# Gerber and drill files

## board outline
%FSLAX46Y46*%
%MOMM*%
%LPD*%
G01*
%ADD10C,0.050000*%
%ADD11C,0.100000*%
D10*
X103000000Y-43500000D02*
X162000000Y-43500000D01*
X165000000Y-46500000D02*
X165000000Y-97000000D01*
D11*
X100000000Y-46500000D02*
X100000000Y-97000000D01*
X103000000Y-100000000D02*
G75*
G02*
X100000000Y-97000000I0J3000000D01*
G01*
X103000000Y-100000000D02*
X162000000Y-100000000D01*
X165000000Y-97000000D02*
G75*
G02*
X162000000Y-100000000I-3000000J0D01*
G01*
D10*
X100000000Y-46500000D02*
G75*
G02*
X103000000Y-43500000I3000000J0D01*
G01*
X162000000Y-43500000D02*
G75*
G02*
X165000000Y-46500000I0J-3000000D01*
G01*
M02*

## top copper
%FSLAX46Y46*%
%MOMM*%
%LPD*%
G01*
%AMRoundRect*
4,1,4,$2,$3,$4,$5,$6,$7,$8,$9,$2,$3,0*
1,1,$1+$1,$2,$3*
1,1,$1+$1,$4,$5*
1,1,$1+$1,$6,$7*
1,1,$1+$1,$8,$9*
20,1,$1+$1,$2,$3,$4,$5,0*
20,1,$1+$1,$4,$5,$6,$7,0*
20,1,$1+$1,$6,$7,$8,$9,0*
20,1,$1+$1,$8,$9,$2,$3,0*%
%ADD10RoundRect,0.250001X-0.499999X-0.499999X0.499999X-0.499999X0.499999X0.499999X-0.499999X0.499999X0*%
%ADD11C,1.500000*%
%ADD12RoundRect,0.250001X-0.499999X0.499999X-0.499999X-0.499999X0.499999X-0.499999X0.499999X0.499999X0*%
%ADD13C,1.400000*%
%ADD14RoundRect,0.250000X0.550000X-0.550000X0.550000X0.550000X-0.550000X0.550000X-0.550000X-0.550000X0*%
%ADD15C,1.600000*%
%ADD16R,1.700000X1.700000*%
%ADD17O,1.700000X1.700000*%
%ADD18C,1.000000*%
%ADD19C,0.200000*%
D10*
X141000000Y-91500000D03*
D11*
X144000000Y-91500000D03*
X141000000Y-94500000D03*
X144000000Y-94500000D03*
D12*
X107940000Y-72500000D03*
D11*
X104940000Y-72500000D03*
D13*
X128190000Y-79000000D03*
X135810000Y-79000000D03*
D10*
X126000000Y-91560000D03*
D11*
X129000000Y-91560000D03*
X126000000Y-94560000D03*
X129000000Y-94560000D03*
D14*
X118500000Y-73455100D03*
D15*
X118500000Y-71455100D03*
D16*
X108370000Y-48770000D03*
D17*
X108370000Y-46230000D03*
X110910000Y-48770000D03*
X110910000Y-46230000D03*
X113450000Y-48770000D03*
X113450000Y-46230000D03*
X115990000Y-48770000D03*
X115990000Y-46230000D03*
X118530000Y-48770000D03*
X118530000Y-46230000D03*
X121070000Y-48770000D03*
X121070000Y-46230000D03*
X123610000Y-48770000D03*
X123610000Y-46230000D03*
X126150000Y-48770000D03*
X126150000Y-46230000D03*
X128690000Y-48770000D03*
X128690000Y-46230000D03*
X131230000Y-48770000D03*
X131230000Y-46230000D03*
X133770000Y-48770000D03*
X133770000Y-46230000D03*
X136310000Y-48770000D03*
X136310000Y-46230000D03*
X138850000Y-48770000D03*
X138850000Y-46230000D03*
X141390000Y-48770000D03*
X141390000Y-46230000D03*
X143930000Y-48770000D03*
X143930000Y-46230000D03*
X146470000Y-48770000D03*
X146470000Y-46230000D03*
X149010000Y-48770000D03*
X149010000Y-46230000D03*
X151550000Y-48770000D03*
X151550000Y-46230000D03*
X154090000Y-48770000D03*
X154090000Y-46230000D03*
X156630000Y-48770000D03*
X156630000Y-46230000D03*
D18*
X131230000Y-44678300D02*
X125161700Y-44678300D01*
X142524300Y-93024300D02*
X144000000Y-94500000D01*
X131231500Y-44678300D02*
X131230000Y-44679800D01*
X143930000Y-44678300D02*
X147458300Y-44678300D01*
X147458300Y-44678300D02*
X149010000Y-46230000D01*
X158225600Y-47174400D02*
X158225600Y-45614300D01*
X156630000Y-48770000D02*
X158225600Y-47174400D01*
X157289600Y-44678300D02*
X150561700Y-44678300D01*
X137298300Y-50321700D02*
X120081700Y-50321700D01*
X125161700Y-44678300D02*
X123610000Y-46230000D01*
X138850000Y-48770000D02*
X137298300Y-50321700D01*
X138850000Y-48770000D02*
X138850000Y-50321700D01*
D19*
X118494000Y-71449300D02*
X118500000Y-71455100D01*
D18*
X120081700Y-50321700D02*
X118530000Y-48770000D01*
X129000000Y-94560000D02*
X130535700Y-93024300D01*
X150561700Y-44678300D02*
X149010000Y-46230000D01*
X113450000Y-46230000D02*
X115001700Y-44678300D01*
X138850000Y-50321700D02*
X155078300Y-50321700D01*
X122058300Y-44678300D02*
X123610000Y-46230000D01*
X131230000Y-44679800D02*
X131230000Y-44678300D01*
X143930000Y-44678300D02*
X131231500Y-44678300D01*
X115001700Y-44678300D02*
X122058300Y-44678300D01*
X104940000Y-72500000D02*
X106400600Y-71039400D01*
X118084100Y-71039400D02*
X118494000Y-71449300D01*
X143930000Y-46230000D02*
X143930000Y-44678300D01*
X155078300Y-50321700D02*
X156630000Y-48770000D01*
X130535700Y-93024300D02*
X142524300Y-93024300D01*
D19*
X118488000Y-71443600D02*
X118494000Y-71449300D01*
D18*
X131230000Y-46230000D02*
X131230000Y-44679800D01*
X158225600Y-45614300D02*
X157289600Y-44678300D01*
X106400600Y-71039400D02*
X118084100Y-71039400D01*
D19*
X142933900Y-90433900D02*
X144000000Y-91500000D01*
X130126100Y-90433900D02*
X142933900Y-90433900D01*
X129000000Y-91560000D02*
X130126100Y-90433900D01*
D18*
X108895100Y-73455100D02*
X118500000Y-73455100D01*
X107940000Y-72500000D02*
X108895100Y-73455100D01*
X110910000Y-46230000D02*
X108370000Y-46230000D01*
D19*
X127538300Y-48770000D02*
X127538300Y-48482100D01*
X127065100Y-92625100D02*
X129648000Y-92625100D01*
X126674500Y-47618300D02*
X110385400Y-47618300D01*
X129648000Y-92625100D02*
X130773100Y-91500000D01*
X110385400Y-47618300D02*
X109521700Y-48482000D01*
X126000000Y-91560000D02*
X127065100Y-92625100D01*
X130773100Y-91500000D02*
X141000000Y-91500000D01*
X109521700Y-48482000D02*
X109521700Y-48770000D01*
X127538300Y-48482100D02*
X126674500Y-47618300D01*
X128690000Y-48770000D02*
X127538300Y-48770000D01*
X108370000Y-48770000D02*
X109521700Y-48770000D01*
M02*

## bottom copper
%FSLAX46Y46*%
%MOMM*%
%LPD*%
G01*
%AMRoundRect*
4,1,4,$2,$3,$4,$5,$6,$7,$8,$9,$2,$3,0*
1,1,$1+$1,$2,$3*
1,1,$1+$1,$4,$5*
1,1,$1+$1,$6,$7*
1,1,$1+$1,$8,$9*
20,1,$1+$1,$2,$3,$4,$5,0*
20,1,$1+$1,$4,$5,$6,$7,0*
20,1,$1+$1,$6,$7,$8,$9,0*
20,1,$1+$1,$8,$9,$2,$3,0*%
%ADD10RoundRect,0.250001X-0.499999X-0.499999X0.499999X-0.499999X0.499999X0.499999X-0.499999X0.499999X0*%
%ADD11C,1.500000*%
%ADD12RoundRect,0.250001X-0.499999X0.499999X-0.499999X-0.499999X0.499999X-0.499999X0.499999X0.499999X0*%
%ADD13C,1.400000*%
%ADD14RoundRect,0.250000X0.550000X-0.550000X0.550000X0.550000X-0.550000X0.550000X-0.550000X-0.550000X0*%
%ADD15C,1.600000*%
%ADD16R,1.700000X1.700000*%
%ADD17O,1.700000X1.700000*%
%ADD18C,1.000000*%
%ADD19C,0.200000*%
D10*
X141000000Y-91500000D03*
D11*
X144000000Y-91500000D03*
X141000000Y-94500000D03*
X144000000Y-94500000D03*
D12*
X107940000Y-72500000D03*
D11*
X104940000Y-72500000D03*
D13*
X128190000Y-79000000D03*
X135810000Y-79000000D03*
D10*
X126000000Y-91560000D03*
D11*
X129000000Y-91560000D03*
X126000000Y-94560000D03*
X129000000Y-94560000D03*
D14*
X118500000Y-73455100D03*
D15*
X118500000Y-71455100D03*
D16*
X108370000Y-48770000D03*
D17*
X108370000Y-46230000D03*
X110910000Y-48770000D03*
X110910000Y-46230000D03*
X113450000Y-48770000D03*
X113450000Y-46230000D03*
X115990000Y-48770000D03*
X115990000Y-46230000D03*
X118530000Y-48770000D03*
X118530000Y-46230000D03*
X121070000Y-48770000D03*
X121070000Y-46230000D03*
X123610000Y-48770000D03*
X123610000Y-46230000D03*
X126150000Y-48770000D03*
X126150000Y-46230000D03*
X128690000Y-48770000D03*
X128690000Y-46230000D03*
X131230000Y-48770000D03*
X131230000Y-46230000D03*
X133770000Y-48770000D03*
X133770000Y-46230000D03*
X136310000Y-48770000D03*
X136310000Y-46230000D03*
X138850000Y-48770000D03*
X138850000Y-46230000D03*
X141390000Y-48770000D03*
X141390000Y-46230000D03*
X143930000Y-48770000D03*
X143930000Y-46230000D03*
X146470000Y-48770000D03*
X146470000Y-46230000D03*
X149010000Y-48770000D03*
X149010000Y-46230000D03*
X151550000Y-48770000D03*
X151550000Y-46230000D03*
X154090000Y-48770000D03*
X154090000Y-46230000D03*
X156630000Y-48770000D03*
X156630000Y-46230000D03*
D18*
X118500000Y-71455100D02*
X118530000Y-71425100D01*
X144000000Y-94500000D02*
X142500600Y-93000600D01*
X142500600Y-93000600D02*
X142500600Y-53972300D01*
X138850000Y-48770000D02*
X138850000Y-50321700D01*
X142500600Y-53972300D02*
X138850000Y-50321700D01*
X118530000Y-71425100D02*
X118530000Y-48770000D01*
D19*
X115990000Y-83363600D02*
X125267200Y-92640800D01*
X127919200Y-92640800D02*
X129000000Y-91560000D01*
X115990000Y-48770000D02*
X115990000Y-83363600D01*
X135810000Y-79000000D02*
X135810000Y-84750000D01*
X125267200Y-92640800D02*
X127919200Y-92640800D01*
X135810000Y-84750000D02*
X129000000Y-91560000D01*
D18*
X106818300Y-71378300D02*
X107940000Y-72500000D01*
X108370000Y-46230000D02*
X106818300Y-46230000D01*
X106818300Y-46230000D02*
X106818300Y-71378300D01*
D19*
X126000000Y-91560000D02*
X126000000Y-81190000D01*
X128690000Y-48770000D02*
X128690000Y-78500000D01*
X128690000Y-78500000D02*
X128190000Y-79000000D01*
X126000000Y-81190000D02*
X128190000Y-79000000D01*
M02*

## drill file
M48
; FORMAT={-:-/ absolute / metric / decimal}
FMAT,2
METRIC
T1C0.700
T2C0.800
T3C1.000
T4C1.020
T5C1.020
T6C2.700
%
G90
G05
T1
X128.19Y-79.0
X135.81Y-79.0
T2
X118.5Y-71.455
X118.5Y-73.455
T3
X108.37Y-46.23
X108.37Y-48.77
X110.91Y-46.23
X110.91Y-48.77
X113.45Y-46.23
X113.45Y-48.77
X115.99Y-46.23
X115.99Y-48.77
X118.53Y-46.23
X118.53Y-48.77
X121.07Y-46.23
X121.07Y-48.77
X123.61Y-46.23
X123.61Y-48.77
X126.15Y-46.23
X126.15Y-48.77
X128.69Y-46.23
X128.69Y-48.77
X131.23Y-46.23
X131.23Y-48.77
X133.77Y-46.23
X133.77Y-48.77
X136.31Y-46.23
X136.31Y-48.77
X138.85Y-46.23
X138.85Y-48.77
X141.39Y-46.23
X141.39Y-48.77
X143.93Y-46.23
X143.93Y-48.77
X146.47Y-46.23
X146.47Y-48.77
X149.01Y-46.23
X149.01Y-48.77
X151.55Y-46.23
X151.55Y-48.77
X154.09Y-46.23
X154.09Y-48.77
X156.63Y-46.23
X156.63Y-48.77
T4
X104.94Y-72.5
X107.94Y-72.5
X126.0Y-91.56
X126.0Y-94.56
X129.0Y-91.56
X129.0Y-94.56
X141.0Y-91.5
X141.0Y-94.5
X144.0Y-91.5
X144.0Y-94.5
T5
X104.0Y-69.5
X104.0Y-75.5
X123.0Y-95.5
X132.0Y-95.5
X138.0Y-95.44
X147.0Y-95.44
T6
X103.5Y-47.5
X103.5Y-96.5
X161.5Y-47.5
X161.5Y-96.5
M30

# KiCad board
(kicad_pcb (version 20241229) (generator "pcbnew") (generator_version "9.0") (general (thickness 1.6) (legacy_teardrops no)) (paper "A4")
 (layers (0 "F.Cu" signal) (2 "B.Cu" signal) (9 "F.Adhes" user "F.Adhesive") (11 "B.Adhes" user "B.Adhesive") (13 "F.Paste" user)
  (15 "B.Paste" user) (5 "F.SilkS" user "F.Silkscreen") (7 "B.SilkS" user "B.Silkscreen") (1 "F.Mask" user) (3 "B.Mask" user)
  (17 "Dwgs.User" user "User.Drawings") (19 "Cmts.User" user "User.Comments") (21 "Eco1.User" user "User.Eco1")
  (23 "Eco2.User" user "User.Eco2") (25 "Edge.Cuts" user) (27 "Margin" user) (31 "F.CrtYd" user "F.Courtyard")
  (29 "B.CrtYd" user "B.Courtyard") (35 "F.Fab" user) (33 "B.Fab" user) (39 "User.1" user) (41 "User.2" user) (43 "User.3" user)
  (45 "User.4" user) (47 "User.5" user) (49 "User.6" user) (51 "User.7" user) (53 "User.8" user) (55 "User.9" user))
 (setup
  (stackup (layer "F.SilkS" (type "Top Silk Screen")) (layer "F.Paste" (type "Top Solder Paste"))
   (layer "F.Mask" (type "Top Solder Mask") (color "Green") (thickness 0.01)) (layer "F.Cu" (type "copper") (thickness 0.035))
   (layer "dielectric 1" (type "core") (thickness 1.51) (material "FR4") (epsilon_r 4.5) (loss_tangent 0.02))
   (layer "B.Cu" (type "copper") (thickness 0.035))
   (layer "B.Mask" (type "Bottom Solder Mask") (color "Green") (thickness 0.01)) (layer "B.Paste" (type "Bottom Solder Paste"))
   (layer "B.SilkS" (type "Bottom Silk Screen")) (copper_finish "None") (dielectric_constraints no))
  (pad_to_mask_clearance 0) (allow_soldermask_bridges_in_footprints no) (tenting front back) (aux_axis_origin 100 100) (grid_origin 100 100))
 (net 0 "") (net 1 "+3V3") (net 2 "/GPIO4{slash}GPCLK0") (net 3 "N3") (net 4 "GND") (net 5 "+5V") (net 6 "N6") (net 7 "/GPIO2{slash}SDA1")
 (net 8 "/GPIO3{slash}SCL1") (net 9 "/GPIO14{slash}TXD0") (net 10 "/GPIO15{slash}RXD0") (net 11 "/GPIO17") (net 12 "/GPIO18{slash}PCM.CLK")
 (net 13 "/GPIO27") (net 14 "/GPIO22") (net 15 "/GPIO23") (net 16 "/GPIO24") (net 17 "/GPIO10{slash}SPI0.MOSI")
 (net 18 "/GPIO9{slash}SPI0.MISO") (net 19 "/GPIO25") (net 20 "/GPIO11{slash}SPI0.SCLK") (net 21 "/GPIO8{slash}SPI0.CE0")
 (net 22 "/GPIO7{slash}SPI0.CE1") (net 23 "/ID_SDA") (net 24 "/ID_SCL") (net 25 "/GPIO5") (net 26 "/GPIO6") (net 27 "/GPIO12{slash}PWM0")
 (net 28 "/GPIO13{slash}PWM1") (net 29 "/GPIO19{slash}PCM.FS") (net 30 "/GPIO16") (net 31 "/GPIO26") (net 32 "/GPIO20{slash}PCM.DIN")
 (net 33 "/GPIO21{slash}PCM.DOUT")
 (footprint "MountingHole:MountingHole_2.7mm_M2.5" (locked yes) (layer "F.Cu") (at 161.5 47.5)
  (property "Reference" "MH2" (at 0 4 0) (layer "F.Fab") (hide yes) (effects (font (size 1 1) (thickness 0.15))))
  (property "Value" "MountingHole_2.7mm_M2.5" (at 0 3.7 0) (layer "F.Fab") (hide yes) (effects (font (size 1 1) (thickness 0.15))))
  (pad "" np_thru_hole circle (at 0 0) (size 2.7 2.7) (drill 2.7) (layers "*.Cu" "*.Mask")))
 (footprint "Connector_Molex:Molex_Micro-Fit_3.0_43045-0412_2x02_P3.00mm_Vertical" (layer "F.Cu") (at 141 91.5)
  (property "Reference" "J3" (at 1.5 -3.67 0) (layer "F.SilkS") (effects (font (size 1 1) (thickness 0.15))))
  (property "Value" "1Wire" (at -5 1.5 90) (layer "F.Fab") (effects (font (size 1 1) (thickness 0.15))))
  (pad "" np_thru_hole circle (at -3 3.94) (size 1.02 1.02) (drill 1.02) (layers "*.Cu" "*.Mask"))
  (pad "" np_thru_hole circle (at 6 3.94) (size 1.02 1.02) (drill 1.02) (layers "*.Cu" "*.Mask"))
  (pad "1" thru_hole roundrect (at 0 0) (size 1.5 1.5) (drill 1.02) (layers "*.Cu" "*.Mask") (remove_unused_layers no)
   (roundrect_rratio 0.166667) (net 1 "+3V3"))
  (pad "2" thru_hole circle (at 3 0) (size 1.5 1.5) (drill 1.02) (layers "*.Cu" "*.Mask") (remove_unused_layers no)
   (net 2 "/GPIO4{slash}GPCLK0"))
  (pad "3" thru_hole circle (at 0 3) (size 1.5 1.5) (drill 1.02) (layers "*.Cu" "*.Mask") (remove_unused_layers no) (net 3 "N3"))
  (pad "4" thru_hole circle (at 3 3) (size 1.5 1.5) (drill 1.02) (layers "*.Cu" "*.Mask") (remove_unused_layers no) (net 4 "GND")))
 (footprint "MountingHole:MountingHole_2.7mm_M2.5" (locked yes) (layer "F.Cu") (at 103.5 96.5)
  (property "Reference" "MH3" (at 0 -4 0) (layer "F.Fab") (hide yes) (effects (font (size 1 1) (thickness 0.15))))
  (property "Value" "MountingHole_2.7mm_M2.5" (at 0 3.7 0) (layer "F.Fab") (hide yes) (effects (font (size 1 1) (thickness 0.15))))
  (pad "" np_thru_hole circle (at 0 0) (size 2.7 2.7) (drill 2.7) (layers "*.Cu" "*.Mask")))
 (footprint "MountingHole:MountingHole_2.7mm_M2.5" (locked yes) (layer "F.Cu") (at 103.5 47.5)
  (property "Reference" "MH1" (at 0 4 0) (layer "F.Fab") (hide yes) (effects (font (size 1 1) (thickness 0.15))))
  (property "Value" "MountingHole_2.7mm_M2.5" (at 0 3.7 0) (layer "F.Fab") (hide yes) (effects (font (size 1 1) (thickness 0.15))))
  (pad "" np_thru_hole circle (at 0 0) (size 2.7 2.7) (drill 2.7) (layers "*.Cu" "*.Mask")))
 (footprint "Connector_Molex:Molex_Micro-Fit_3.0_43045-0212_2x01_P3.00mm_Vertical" (layer "F.Cu") (at 107.94 72.5 -90)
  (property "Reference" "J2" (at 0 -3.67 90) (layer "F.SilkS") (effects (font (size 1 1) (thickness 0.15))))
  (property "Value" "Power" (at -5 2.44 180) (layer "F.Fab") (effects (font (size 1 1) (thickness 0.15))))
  (pad "" np_thru_hole circle (at -3 3.94 270) (size 1.02 1.02) (drill 1.02) (layers "*.Cu" "*.Mask"))
  (pad "" np_thru_hole circle (at 3 3.94 270) (size 1.02 1.02) (drill 1.02) (layers "*.Cu" "*.Mask"))
  (pad "1" thru_hole roundrect (at 0 0 270) (size 1.5 1.5) (drill 1.02) (layers "*.Cu" "*.Mask") (remove_unused_layers no)
   (roundrect_rratio 0.166667) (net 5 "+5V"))
  (pad "2" thru_hole circle (at 0 3 270) (size 1.5 1.5) (drill 1.02) (layers "*.Cu" "*.Mask") (remove_unused_layers no) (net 4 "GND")))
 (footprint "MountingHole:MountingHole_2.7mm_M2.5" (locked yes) (layer "F.Cu") (at 161.5 96.5)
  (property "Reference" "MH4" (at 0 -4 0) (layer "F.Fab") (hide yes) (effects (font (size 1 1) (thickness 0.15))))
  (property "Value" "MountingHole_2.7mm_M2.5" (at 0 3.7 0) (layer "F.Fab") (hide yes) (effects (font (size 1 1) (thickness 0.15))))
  (pad "" np_thru_hole circle (at 0 0) (size 2.7 2.7) (drill 2.7) (layers "*.Cu" "*.Mask")))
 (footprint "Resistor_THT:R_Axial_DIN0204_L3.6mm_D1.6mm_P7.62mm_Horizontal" (layer "F.Cu") (at 128.19 79)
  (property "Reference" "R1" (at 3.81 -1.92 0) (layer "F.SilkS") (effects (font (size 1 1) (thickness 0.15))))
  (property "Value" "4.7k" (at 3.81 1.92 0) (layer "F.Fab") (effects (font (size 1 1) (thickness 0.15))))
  (pad "1" thru_hole circle (at 0 0) (size 1.4 1.4) (drill 0.7) (layers "*.Cu" "*.Mask") (remove_unused_layers no) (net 1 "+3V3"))
  (pad "2" thru_hole circle (at 7.62 0) (size 1.4 1.4) (drill 0.7) (layers "*.Cu" "*.Mask") (remove_unused_layers no)
   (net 2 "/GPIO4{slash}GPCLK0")))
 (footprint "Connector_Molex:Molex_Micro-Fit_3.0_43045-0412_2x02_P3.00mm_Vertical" (layer "F.Cu") (at 126 91.56)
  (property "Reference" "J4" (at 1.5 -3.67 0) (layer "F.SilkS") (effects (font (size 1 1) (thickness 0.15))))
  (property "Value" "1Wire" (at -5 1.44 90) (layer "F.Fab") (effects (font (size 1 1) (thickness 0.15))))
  (pad "" np_thru_hole circle (at -3 3.94) (size 1.02 1.02) (drill 1.02) (layers "*.Cu" "*.Mask"))
  (pad "" np_thru_hole circle (at 6 3.94) (size 1.02 1.02) (drill 1.02) (layers "*.Cu" "*.Mask"))
  (pad "1" thru_hole roundrect (at 0 0) (size 1.5 1.5) (drill 1.02) (layers "*.Cu" "*.Mask") (remove_unused_layers no)
   (roundrect_rratio 0.166667) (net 1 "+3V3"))
  (pad "2" thru_hole circle (at 3 0) (size 1.5 1.5) (drill 1.02) (layers "*.Cu" "*.Mask") (remove_unused_layers no)
   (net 2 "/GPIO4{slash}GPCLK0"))
  (pad "3" thru_hole circle (at 0 3) (size 1.5 1.5) (drill 1.02) (layers "*.Cu" "*.Mask") (remove_unused_layers no) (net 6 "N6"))
  (pad "4" thru_hole circle (at 3 3) (size 1.5 1.5) (drill 1.02) (layers "*.Cu" "*.Mask") (remove_unused_layers no) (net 4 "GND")))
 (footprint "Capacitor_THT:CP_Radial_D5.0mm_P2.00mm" (layer "F.Cu") (at 118.5 73.4551 90)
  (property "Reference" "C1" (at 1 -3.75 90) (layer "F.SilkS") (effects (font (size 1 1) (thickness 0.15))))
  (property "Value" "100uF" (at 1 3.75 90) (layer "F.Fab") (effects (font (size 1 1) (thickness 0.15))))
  (pad "1" thru_hole roundrect (at 0 0 90) (size 1.6 1.6) (drill 0.8) (layers "*.Cu" "*.Mask") (remove_unused_layers no)
   (roundrect_rratio 0.15625) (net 5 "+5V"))
  (pad "2" thru_hole circle (at 2 0 90) (size 1.6 1.6) (drill 0.8) (layers "*.Cu" "*.Mask") (remove_unused_layers no) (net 4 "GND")))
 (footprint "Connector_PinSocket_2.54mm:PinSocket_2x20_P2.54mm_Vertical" (layer "B.Cu") (at 108.37 48.77 -90)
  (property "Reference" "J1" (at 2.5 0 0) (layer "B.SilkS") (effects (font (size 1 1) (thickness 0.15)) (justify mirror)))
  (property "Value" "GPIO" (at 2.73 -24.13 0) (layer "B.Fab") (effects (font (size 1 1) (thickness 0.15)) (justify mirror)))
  (pad "1" thru_hole rect (at 0 0 270) (size 1.7 1.7) (drill 1) (layers "*.Cu" "*.Mask") (remove_unused_layers no) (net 1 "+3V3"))
  (pad "2" thru_hole oval (at -2.54 0 270) (size 1.7 1.7) (drill 1) (layers "*.Cu" "*.Mask") (remove_unused_layers no) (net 5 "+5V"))
  (pad "3" thru_hole oval (at 0 -2.54 270) (size 1.7 1.7) (drill 1) (layers "*.Cu" "*.Mask") (remove_unused_layers no)
   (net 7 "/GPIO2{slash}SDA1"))
  (pad "4" thru_hole oval (at -2.54 -2.54 270) (size 1.7 1.7) (drill 1) (layers "*.Cu" "*.Mask") (remove_unused_layers no) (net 5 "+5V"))
  (pad "5" thru_hole oval (at 0 -5.08 270) (size 1.7 1.7) (drill 1) (layers "*.Cu" "*.Mask") (remove_unused_layers no)
   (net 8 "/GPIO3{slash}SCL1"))
  (pad "6" thru_hole oval (at -2.54 -5.08 270) (size 1.7 1.7) (drill 1) (layers "*.Cu" "*.Mask") (remove_unused_layers no) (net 4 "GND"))
  (pad "7" thru_hole oval (at 0 -7.62 270) (size 1.7 1.7) (drill 1) (layers "*.Cu" "*.Mask") (remove_unused_layers no)
   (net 2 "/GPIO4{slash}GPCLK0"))
  (pad "8" thru_hole oval (at -2.54 -7.62 270) (size 1.7 1.7) (drill 1) (layers "*.Cu" "*.Mask") (remove_unused_layers no)
   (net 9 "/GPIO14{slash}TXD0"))
  (pad "9" thru_hole oval (at 0 -10.16 270) (size 1.7 1.7) (drill 1) (layers "*.Cu" "*.Mask") (remove_unused_layers no) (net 4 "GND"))
  (pad "10" thru_hole oval (at -2.54 -10.16 270) (size 1.7 1.7) (drill 1) (layers "*.Cu" "*.Mask") (remove_unused_layers no)
   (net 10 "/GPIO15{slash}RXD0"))
  (pad "11" thru_hole oval (at 0 -12.7 270) (size 1.7 1.7) (drill 1) (layers "*.Cu" "*.Mask") (remove_unused_layers no) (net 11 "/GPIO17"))
  (pad "12" thru_hole oval (at -2.54 -12.7 270) (size 1.7 1.7) (drill 1) (layers "*.Cu" "*.Mask") (remove_unused_layers no)
   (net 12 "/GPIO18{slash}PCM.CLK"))
  (pad "13" thru_hole oval (at 0 -15.24 270) (size 1.7 1.7) (drill 1) (layers "*.Cu" "*.Mask") (remove_unused_layers no) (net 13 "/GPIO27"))
  (pad "14" thru_hole oval (at -2.54 -15.24 270) (size 1.7 1.7) (drill 1) (layers "*.Cu" "*.Mask") (remove_unused_layers no) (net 4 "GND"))
  (pad "15" thru_hole oval (at 0 -17.78 270) (size 1.7 1.7) (drill 1) (layers "*.Cu" "*.Mask") (remove_unused_layers no) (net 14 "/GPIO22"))
  (pad "16" thru_hole oval (at -2.54 -17.78 270) (size 1.7 1.7) (drill 1) (layers "*.Cu" "*.Mask") (remove_unused_layers no)
   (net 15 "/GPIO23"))
  (pad "17" thru_hole oval (at 0 -20.32 270) (size 1.7 1.7) (drill 1) (layers "*.Cu" "*.Mask") (remove_unused_layers no) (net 1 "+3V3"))
  (pad "18" thru_hole oval (at -2.54 -20.32 270) (size 1.7 1.7) (drill 1) (layers "*.Cu" "*.Mask") (remove_unused_layers no)
   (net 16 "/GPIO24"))
  (pad "19" thru_hole oval (at 0 -22.86 270) (size 1.7 1.7) (drill 1) (layers "*.Cu" "*.Mask") (remove_unused_layers no)
   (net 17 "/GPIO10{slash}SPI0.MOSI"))
  (pad "20" thru_hole oval (at -2.54 -22.86 270) (size 1.7 1.7) (drill 1) (layers "*.Cu" "*.Mask") (remove_unused_layers no) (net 4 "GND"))
  (pad "21" thru_hole oval (at 0 -25.4 270) (size 1.7 1.7) (drill 1) (layers "*.Cu" "*.Mask") (remove_unused_layers no)
   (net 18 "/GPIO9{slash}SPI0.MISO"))
  (pad "22" thru_hole oval (at -2.54 -25.4 270) (size 1.7 1.7) (drill 1) (layers "*.Cu" "*.Mask") (remove_unused_layers no)
   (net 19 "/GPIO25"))
  (pad "23" thru_hole oval (at 0 -27.94 270) (size 1.7 1.7) (drill 1) (layers "*.Cu" "*.Mask") (remove_unused_layers no)
   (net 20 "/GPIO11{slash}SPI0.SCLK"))
  (pad "24" thru_hole oval (at -2.54 -27.94 270) (size 1.7 1.7) (drill 1) (layers "*.Cu" "*.Mask") (remove_unused_layers no)
   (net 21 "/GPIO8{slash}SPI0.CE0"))
  (pad "25" thru_hole oval (at 0 -30.48 270) (size 1.7 1.7) (drill 1) (layers "*.Cu" "*.Mask") (remove_unused_layers no) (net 4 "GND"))
  (pad "26" thru_hole oval (at -2.54 -30.48 270) (size 1.7 1.7) (drill 1) (layers "*.Cu" "*.Mask") (remove_unused_layers no)
   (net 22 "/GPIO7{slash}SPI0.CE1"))
  (pad "27" thru_hole oval (at 0 -33.02 270) (size 1.7 1.7) (drill 1) (layers "*.Cu" "*.Mask") (remove_unused_layers no) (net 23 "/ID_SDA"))
  (pad "28" thru_hole oval (at -2.54 -33.02 270) (size 1.7 1.7) (drill 1) (layers "*.Cu" "*.Mask") (remove_unused_layers no)
   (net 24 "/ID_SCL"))
  (pad "29" thru_hole oval (at 0 -35.56 270) (size 1.7 1.7) (drill 1) (layers "*.Cu" "*.Mask") (remove_unused_layers no) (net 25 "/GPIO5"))
  (pad "30" thru_hole oval (at -2.54 -35.56 270) (size 1.7 1.7) (drill 1) (layers "*.Cu" "*.Mask") (remove_unused_layers no) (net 4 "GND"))
  (pad "31" thru_hole oval (at 0 -38.1 270) (size 1.7 1.7) (drill 1) (layers "*.Cu" "*.Mask") (remove_unused_layers no) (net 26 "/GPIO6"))
  (pad "32" thru_hole oval (at -2.54 -38.1 270) (size 1.7 1.7) (drill 1) (layers "*.Cu" "*.Mask") (remove_unused_layers no)
   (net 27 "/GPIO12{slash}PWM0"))
  (pad "33" thru_hole oval (at 0 -40.64 270) (size 1.7 1.7) (drill 1) (layers "*.Cu" "*.Mask") (remove_unused_layers no)
   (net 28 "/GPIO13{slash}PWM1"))
  (pad "34" thru_hole oval (at -2.54 -40.64 270) (size 1.7 1.7) (drill 1) (layers "*.Cu" "*.Mask") (remove_unused_layers no) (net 4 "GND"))
  (pad "35" thru_hole oval (at 0 -43.18 270) (size 1.7 1.7) (drill 1) (layers "*.Cu" "*.Mask") (remove_unused_layers no)
   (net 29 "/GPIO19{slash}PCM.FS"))
  (pad "36" thru_hole oval (at -2.54 -43.18 270) (size 1.7 1.7) (drill 1) (layers "*.Cu" "*.Mask") (remove_unused_layers no)
   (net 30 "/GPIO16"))
  (pad "37" thru_hole oval (at 0 -45.72 270) (size 1.7 1.7) (drill 1) (layers "*.Cu" "*.Mask") (remove_unused_layers no) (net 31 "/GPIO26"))
  (pad "38" thru_hole oval (at -2.54 -45.72 270) (size 1.7 1.7) (drill 1) (layers "*.Cu" "*.Mask") (remove_unused_layers no)
   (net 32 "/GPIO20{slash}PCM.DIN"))
  (pad "39" thru_hole oval (at 0 -48.26 270) (size 1.7 1.7) (drill 1) (layers "*.Cu" "*.Mask") (remove_unused_layers no) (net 4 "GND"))
  (pad "40" thru_hole oval (at -2.54 -48.26 270) (size 1.7 1.7) (drill 1) (layers "*.Cu" "*.Mask") (remove_unused_layers no)
   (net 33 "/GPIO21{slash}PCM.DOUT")))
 (gr_line (start 103 43.5) (end 162 43.5) (stroke (width 0.05) (type default)) (layer "Edge.Cuts"))
 (gr_line (start 165 46.5) (end 165 97) (stroke (width 0.05) (type default)) (layer "Edge.Cuts"))
 (gr_line (start 100 46.5) (end 100 97) (stroke (width 0.1) (type solid)) (layer "Edge.Cuts"))
 (gr_arc (start 103 100) (mid 100.87868 99.12132) (end 100 97) (stroke (width 0.1) (type solid)) (layer "Edge.Cuts"))
 (gr_line (start 103 100) (end 162 100) (stroke (width 0.1) (type solid)) (layer "Edge.Cuts"))
 (gr_arc (start 165 97) (mid 164.12132 99.12132) (end 162 100) (stroke (width 0.1) (type solid)) (layer "Edge.Cuts"))
 (gr_arc (start 100 46.5) (mid 100.87868 44.37868) (end 103 43.5) (stroke (width 0.05) (type default)) (layer "Edge.Cuts"))
 (gr_arc (start 162 43.5) (mid 164.12132 44.37868) (end 165 46.5) (stroke (width 0.05) (type default)) (layer "Edge.Cuts"))
 (segment (start 131.23 44.6783) (end 125.1617 44.6783) (width 1) (layer "F.Cu") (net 4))
 (segment (start 142.5243 93.0243) (end 144 94.5) (width 1) (layer "F.Cu") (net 4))
 (segment (start 131.2315 44.6783) (end 131.23 44.6798) (width 1) (layer "F.Cu") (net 4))
 (segment (start 143.93 44.6783) (end 147.4583 44.6783) (width 1) (layer "F.Cu") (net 4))
 (segment (start 147.4583 44.6783) (end 149.01 46.23) (width 1) (layer "F.Cu") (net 4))
 (segment (start 158.2256 47.1744) (end 158.2256 45.6143) (width 1) (layer "F.Cu") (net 4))
 (segment (start 156.63 48.77) (end 158.2256 47.1744) (width 1) (layer "F.Cu") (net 4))
 (segment (start 157.2896 44.6783) (end 150.5617 44.6783) (width 1) (layer "F.Cu") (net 4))
 (segment (start 137.2983 50.3217) (end 120.0817 50.3217) (width 1) (layer "F.Cu") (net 4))
 (segment (start 125.1617 44.6783) (end 123.61 46.23) (width 1) (layer "F.Cu") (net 4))
 (segment (start 138.85 48.77) (end 137.2983 50.3217) (width 1) (layer "F.Cu") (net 4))
 (segment (start 138.85 48.77) (end 138.85 50.3217) (width 1) (layer "F.Cu") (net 4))
 (segment (start 118.494 71.4493) (end 118.5 71.4551) (width 0.2) (layer "F.Cu") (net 4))
 (segment (start 120.0817 50.3217) (end 118.53 48.77) (width 1) (layer "F.Cu") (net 4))
 (segment (start 129 94.56) (end 130.5357 93.0243) (width 1) (layer "F.Cu") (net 4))
 (segment (start 150.5617 44.6783) (end 149.01 46.23) (width 1) (layer "F.Cu") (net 4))
 (segment (start 113.45 46.23) (end 115.0017 44.6783) (width 1) (layer "F.Cu") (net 4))
 (segment (start 138.85 50.3217) (end 155.0783 50.3217) (width 1) (layer "F.Cu") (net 4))
 (segment (start 122.0583 44.6783) (end 123.61 46.23) (width 1) (layer "F.Cu") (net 4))
 (segment (start 131.23 44.6798) (end 131.23 44.6783) (width 1) (layer "F.Cu") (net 4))
 (segment (start 143.93 44.6783) (end 131.2315 44.6783) (width 1) (layer "F.Cu") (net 4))
 (segment (start 115.0017 44.6783) (end 122.0583 44.6783) (width 1) (layer "F.Cu") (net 4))
 (segment (start 104.94 72.5) (end 106.4006 71.0394) (width 1) (layer "F.Cu") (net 4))
 (segment (start 118.0841 71.0394) (end 118.494 71.4493) (width 1) (layer "F.Cu") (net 4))
 (segment (start 143.93 46.23) (end 143.93 44.6783) (width 1) (layer "F.Cu") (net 4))
 (segment (start 155.0783 50.3217) (end 156.63 48.77) (width 1) (layer "F.Cu") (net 4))
 (segment (start 130.5357 93.0243) (end 142.5243 93.0243) (width 1) (layer "F.Cu") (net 4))
 (segment (start 118.488 71.4436) (end 118.494 71.4493) (width 0.2) (layer "F.Cu") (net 4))
 (segment (start 131.23 46.23) (end 131.23 44.6798) (width 1) (layer "F.Cu") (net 4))
 (segment (start 158.2256 45.6143) (end 157.2896 44.6783) (width 1) (layer "F.Cu") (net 4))
 (segment (start 106.4006 71.0394) (end 118.0841 71.0394) (width 1) (layer "F.Cu") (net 4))
 (segment (start 118.5 71.4551) (end 118.53 71.4251) (width 1) (layer "B.Cu") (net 4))
 (segment (start 144 94.5) (end 142.5006 93.0006) (width 1) (layer "B.Cu") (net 4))
 (segment (start 142.5006 93.0006) (end 142.5006 53.9723) (width 1) (layer "B.Cu") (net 4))
 (segment (start 138.85 48.77) (end 138.85 50.3217) (width 1) (layer "B.Cu") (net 4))
 (segment (start 142.5006 53.9723) (end 138.85 50.3217) (width 1) (layer "B.Cu") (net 4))
 (segment (start 118.53 71.4251) (end 118.53 48.77) (width 1) (layer "B.Cu") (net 4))
 (segment (start 142.9339 90.4339) (end 144 91.5) (width 0.2) (layer "F.Cu") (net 2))
 (segment (start 130.1261 90.4339) (end 142.9339 90.4339) (width 0.2) (layer "F.Cu") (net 2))
 (segment (start 129 91.56) (end 130.1261 90.4339) (width 0.2) (layer "F.Cu") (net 2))
 (segment (start 115.99 83.3636) (end 125.2672 92.6408) (width 0.2) (layer "B.Cu") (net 2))
 (segment (start 127.9192 92.6408) (end 129 91.56) (width 0.2) (layer "B.Cu") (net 2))
 (segment (start 115.99 48.77) (end 115.99 83.3636) (width 0.2) (layer "B.Cu") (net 2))
 (segment (start 135.81 79) (end 135.81 84.75) (width 0.2) (layer "B.Cu") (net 2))
 (segment (start 125.2672 92.6408) (end 127.9192 92.6408) (width 0.2) (layer "B.Cu") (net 2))
 (segment (start 135.81 84.75) (end 129 91.56) (width 0.2) (layer "B.Cu") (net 2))
 (segment (start 108.8951 73.4551) (end 118.5 73.4551) (width 1) (layer "F.Cu") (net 5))
 (segment (start 107.94 72.5) (end 108.8951 73.4551) (width 1) (layer "F.Cu") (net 5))
 (segment (start 110.91 46.23) (end 108.37 46.23) (width 1) (layer "F.Cu") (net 5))
 (segment (start 106.8183 71.3783) (end 107.94 72.5) (width 1) (layer "B.Cu") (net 5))
 (segment (start 108.37 46.23) (end 106.8183 46.23) (width 1) (layer "B.Cu") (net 5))
 (segment (start 106.8183 46.23) (end 106.8183 71.3783) (width 1) (layer "B.Cu") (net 5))
 (segment (start 127.5383 48.77) (end 127.5383 48.4821) (width 0.2) (layer "F.Cu") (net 1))
 (segment (start 127.0651 92.6251) (end 129.648 92.6251) (width 0.2) (layer "F.Cu") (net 1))
 (segment (start 126.6745 47.6183) (end 110.3854 47.6183) (width 0.2) (layer "F.Cu") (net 1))
 (segment (start 129.648 92.6251) (end 130.7731 91.5) (width 0.2) (layer "F.Cu") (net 1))
 (segment (start 110.3854 47.6183) (end 109.5217 48.482) (width 0.2) (layer "F.Cu") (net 1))
 (segment (start 126 91.56) (end 127.0651 92.6251) (width 0.2) (layer "F.Cu") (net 1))
 (segment (start 130.7731 91.5) (end 141 91.5) (width 0.2) (layer "F.Cu") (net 1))
 (segment (start 109.5217 48.482) (end 109.5217 48.77) (width 0.2) (layer "F.Cu") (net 1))
 (segment (start 127.5383 48.4821) (end 126.6745 47.6183) (width 0.2) (layer "F.Cu") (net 1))
 (segment (start 128.69 48.77) (end 127.5383 48.77) (width 0.2) (layer "F.Cu") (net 1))
 (segment (start 108.37 48.77) (end 109.5217 48.77) (width 0.2) (layer "F.Cu") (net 1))
 (segment (start 126 91.56) (end 126 81.19) (width 0.2) (layer "B.Cu") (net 1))
 (segment (start 128.69 48.77) (end 128.69 78.5) (width 0.2) (layer "B.Cu") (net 1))
 (segment (start 128.69 78.5) (end 128.19 79) (width 0.2) (layer "B.Cu") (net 1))
 (segment (start 126 81.19) (end 128.19 79) (width 0.2) (layer "B.Cu") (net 1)))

